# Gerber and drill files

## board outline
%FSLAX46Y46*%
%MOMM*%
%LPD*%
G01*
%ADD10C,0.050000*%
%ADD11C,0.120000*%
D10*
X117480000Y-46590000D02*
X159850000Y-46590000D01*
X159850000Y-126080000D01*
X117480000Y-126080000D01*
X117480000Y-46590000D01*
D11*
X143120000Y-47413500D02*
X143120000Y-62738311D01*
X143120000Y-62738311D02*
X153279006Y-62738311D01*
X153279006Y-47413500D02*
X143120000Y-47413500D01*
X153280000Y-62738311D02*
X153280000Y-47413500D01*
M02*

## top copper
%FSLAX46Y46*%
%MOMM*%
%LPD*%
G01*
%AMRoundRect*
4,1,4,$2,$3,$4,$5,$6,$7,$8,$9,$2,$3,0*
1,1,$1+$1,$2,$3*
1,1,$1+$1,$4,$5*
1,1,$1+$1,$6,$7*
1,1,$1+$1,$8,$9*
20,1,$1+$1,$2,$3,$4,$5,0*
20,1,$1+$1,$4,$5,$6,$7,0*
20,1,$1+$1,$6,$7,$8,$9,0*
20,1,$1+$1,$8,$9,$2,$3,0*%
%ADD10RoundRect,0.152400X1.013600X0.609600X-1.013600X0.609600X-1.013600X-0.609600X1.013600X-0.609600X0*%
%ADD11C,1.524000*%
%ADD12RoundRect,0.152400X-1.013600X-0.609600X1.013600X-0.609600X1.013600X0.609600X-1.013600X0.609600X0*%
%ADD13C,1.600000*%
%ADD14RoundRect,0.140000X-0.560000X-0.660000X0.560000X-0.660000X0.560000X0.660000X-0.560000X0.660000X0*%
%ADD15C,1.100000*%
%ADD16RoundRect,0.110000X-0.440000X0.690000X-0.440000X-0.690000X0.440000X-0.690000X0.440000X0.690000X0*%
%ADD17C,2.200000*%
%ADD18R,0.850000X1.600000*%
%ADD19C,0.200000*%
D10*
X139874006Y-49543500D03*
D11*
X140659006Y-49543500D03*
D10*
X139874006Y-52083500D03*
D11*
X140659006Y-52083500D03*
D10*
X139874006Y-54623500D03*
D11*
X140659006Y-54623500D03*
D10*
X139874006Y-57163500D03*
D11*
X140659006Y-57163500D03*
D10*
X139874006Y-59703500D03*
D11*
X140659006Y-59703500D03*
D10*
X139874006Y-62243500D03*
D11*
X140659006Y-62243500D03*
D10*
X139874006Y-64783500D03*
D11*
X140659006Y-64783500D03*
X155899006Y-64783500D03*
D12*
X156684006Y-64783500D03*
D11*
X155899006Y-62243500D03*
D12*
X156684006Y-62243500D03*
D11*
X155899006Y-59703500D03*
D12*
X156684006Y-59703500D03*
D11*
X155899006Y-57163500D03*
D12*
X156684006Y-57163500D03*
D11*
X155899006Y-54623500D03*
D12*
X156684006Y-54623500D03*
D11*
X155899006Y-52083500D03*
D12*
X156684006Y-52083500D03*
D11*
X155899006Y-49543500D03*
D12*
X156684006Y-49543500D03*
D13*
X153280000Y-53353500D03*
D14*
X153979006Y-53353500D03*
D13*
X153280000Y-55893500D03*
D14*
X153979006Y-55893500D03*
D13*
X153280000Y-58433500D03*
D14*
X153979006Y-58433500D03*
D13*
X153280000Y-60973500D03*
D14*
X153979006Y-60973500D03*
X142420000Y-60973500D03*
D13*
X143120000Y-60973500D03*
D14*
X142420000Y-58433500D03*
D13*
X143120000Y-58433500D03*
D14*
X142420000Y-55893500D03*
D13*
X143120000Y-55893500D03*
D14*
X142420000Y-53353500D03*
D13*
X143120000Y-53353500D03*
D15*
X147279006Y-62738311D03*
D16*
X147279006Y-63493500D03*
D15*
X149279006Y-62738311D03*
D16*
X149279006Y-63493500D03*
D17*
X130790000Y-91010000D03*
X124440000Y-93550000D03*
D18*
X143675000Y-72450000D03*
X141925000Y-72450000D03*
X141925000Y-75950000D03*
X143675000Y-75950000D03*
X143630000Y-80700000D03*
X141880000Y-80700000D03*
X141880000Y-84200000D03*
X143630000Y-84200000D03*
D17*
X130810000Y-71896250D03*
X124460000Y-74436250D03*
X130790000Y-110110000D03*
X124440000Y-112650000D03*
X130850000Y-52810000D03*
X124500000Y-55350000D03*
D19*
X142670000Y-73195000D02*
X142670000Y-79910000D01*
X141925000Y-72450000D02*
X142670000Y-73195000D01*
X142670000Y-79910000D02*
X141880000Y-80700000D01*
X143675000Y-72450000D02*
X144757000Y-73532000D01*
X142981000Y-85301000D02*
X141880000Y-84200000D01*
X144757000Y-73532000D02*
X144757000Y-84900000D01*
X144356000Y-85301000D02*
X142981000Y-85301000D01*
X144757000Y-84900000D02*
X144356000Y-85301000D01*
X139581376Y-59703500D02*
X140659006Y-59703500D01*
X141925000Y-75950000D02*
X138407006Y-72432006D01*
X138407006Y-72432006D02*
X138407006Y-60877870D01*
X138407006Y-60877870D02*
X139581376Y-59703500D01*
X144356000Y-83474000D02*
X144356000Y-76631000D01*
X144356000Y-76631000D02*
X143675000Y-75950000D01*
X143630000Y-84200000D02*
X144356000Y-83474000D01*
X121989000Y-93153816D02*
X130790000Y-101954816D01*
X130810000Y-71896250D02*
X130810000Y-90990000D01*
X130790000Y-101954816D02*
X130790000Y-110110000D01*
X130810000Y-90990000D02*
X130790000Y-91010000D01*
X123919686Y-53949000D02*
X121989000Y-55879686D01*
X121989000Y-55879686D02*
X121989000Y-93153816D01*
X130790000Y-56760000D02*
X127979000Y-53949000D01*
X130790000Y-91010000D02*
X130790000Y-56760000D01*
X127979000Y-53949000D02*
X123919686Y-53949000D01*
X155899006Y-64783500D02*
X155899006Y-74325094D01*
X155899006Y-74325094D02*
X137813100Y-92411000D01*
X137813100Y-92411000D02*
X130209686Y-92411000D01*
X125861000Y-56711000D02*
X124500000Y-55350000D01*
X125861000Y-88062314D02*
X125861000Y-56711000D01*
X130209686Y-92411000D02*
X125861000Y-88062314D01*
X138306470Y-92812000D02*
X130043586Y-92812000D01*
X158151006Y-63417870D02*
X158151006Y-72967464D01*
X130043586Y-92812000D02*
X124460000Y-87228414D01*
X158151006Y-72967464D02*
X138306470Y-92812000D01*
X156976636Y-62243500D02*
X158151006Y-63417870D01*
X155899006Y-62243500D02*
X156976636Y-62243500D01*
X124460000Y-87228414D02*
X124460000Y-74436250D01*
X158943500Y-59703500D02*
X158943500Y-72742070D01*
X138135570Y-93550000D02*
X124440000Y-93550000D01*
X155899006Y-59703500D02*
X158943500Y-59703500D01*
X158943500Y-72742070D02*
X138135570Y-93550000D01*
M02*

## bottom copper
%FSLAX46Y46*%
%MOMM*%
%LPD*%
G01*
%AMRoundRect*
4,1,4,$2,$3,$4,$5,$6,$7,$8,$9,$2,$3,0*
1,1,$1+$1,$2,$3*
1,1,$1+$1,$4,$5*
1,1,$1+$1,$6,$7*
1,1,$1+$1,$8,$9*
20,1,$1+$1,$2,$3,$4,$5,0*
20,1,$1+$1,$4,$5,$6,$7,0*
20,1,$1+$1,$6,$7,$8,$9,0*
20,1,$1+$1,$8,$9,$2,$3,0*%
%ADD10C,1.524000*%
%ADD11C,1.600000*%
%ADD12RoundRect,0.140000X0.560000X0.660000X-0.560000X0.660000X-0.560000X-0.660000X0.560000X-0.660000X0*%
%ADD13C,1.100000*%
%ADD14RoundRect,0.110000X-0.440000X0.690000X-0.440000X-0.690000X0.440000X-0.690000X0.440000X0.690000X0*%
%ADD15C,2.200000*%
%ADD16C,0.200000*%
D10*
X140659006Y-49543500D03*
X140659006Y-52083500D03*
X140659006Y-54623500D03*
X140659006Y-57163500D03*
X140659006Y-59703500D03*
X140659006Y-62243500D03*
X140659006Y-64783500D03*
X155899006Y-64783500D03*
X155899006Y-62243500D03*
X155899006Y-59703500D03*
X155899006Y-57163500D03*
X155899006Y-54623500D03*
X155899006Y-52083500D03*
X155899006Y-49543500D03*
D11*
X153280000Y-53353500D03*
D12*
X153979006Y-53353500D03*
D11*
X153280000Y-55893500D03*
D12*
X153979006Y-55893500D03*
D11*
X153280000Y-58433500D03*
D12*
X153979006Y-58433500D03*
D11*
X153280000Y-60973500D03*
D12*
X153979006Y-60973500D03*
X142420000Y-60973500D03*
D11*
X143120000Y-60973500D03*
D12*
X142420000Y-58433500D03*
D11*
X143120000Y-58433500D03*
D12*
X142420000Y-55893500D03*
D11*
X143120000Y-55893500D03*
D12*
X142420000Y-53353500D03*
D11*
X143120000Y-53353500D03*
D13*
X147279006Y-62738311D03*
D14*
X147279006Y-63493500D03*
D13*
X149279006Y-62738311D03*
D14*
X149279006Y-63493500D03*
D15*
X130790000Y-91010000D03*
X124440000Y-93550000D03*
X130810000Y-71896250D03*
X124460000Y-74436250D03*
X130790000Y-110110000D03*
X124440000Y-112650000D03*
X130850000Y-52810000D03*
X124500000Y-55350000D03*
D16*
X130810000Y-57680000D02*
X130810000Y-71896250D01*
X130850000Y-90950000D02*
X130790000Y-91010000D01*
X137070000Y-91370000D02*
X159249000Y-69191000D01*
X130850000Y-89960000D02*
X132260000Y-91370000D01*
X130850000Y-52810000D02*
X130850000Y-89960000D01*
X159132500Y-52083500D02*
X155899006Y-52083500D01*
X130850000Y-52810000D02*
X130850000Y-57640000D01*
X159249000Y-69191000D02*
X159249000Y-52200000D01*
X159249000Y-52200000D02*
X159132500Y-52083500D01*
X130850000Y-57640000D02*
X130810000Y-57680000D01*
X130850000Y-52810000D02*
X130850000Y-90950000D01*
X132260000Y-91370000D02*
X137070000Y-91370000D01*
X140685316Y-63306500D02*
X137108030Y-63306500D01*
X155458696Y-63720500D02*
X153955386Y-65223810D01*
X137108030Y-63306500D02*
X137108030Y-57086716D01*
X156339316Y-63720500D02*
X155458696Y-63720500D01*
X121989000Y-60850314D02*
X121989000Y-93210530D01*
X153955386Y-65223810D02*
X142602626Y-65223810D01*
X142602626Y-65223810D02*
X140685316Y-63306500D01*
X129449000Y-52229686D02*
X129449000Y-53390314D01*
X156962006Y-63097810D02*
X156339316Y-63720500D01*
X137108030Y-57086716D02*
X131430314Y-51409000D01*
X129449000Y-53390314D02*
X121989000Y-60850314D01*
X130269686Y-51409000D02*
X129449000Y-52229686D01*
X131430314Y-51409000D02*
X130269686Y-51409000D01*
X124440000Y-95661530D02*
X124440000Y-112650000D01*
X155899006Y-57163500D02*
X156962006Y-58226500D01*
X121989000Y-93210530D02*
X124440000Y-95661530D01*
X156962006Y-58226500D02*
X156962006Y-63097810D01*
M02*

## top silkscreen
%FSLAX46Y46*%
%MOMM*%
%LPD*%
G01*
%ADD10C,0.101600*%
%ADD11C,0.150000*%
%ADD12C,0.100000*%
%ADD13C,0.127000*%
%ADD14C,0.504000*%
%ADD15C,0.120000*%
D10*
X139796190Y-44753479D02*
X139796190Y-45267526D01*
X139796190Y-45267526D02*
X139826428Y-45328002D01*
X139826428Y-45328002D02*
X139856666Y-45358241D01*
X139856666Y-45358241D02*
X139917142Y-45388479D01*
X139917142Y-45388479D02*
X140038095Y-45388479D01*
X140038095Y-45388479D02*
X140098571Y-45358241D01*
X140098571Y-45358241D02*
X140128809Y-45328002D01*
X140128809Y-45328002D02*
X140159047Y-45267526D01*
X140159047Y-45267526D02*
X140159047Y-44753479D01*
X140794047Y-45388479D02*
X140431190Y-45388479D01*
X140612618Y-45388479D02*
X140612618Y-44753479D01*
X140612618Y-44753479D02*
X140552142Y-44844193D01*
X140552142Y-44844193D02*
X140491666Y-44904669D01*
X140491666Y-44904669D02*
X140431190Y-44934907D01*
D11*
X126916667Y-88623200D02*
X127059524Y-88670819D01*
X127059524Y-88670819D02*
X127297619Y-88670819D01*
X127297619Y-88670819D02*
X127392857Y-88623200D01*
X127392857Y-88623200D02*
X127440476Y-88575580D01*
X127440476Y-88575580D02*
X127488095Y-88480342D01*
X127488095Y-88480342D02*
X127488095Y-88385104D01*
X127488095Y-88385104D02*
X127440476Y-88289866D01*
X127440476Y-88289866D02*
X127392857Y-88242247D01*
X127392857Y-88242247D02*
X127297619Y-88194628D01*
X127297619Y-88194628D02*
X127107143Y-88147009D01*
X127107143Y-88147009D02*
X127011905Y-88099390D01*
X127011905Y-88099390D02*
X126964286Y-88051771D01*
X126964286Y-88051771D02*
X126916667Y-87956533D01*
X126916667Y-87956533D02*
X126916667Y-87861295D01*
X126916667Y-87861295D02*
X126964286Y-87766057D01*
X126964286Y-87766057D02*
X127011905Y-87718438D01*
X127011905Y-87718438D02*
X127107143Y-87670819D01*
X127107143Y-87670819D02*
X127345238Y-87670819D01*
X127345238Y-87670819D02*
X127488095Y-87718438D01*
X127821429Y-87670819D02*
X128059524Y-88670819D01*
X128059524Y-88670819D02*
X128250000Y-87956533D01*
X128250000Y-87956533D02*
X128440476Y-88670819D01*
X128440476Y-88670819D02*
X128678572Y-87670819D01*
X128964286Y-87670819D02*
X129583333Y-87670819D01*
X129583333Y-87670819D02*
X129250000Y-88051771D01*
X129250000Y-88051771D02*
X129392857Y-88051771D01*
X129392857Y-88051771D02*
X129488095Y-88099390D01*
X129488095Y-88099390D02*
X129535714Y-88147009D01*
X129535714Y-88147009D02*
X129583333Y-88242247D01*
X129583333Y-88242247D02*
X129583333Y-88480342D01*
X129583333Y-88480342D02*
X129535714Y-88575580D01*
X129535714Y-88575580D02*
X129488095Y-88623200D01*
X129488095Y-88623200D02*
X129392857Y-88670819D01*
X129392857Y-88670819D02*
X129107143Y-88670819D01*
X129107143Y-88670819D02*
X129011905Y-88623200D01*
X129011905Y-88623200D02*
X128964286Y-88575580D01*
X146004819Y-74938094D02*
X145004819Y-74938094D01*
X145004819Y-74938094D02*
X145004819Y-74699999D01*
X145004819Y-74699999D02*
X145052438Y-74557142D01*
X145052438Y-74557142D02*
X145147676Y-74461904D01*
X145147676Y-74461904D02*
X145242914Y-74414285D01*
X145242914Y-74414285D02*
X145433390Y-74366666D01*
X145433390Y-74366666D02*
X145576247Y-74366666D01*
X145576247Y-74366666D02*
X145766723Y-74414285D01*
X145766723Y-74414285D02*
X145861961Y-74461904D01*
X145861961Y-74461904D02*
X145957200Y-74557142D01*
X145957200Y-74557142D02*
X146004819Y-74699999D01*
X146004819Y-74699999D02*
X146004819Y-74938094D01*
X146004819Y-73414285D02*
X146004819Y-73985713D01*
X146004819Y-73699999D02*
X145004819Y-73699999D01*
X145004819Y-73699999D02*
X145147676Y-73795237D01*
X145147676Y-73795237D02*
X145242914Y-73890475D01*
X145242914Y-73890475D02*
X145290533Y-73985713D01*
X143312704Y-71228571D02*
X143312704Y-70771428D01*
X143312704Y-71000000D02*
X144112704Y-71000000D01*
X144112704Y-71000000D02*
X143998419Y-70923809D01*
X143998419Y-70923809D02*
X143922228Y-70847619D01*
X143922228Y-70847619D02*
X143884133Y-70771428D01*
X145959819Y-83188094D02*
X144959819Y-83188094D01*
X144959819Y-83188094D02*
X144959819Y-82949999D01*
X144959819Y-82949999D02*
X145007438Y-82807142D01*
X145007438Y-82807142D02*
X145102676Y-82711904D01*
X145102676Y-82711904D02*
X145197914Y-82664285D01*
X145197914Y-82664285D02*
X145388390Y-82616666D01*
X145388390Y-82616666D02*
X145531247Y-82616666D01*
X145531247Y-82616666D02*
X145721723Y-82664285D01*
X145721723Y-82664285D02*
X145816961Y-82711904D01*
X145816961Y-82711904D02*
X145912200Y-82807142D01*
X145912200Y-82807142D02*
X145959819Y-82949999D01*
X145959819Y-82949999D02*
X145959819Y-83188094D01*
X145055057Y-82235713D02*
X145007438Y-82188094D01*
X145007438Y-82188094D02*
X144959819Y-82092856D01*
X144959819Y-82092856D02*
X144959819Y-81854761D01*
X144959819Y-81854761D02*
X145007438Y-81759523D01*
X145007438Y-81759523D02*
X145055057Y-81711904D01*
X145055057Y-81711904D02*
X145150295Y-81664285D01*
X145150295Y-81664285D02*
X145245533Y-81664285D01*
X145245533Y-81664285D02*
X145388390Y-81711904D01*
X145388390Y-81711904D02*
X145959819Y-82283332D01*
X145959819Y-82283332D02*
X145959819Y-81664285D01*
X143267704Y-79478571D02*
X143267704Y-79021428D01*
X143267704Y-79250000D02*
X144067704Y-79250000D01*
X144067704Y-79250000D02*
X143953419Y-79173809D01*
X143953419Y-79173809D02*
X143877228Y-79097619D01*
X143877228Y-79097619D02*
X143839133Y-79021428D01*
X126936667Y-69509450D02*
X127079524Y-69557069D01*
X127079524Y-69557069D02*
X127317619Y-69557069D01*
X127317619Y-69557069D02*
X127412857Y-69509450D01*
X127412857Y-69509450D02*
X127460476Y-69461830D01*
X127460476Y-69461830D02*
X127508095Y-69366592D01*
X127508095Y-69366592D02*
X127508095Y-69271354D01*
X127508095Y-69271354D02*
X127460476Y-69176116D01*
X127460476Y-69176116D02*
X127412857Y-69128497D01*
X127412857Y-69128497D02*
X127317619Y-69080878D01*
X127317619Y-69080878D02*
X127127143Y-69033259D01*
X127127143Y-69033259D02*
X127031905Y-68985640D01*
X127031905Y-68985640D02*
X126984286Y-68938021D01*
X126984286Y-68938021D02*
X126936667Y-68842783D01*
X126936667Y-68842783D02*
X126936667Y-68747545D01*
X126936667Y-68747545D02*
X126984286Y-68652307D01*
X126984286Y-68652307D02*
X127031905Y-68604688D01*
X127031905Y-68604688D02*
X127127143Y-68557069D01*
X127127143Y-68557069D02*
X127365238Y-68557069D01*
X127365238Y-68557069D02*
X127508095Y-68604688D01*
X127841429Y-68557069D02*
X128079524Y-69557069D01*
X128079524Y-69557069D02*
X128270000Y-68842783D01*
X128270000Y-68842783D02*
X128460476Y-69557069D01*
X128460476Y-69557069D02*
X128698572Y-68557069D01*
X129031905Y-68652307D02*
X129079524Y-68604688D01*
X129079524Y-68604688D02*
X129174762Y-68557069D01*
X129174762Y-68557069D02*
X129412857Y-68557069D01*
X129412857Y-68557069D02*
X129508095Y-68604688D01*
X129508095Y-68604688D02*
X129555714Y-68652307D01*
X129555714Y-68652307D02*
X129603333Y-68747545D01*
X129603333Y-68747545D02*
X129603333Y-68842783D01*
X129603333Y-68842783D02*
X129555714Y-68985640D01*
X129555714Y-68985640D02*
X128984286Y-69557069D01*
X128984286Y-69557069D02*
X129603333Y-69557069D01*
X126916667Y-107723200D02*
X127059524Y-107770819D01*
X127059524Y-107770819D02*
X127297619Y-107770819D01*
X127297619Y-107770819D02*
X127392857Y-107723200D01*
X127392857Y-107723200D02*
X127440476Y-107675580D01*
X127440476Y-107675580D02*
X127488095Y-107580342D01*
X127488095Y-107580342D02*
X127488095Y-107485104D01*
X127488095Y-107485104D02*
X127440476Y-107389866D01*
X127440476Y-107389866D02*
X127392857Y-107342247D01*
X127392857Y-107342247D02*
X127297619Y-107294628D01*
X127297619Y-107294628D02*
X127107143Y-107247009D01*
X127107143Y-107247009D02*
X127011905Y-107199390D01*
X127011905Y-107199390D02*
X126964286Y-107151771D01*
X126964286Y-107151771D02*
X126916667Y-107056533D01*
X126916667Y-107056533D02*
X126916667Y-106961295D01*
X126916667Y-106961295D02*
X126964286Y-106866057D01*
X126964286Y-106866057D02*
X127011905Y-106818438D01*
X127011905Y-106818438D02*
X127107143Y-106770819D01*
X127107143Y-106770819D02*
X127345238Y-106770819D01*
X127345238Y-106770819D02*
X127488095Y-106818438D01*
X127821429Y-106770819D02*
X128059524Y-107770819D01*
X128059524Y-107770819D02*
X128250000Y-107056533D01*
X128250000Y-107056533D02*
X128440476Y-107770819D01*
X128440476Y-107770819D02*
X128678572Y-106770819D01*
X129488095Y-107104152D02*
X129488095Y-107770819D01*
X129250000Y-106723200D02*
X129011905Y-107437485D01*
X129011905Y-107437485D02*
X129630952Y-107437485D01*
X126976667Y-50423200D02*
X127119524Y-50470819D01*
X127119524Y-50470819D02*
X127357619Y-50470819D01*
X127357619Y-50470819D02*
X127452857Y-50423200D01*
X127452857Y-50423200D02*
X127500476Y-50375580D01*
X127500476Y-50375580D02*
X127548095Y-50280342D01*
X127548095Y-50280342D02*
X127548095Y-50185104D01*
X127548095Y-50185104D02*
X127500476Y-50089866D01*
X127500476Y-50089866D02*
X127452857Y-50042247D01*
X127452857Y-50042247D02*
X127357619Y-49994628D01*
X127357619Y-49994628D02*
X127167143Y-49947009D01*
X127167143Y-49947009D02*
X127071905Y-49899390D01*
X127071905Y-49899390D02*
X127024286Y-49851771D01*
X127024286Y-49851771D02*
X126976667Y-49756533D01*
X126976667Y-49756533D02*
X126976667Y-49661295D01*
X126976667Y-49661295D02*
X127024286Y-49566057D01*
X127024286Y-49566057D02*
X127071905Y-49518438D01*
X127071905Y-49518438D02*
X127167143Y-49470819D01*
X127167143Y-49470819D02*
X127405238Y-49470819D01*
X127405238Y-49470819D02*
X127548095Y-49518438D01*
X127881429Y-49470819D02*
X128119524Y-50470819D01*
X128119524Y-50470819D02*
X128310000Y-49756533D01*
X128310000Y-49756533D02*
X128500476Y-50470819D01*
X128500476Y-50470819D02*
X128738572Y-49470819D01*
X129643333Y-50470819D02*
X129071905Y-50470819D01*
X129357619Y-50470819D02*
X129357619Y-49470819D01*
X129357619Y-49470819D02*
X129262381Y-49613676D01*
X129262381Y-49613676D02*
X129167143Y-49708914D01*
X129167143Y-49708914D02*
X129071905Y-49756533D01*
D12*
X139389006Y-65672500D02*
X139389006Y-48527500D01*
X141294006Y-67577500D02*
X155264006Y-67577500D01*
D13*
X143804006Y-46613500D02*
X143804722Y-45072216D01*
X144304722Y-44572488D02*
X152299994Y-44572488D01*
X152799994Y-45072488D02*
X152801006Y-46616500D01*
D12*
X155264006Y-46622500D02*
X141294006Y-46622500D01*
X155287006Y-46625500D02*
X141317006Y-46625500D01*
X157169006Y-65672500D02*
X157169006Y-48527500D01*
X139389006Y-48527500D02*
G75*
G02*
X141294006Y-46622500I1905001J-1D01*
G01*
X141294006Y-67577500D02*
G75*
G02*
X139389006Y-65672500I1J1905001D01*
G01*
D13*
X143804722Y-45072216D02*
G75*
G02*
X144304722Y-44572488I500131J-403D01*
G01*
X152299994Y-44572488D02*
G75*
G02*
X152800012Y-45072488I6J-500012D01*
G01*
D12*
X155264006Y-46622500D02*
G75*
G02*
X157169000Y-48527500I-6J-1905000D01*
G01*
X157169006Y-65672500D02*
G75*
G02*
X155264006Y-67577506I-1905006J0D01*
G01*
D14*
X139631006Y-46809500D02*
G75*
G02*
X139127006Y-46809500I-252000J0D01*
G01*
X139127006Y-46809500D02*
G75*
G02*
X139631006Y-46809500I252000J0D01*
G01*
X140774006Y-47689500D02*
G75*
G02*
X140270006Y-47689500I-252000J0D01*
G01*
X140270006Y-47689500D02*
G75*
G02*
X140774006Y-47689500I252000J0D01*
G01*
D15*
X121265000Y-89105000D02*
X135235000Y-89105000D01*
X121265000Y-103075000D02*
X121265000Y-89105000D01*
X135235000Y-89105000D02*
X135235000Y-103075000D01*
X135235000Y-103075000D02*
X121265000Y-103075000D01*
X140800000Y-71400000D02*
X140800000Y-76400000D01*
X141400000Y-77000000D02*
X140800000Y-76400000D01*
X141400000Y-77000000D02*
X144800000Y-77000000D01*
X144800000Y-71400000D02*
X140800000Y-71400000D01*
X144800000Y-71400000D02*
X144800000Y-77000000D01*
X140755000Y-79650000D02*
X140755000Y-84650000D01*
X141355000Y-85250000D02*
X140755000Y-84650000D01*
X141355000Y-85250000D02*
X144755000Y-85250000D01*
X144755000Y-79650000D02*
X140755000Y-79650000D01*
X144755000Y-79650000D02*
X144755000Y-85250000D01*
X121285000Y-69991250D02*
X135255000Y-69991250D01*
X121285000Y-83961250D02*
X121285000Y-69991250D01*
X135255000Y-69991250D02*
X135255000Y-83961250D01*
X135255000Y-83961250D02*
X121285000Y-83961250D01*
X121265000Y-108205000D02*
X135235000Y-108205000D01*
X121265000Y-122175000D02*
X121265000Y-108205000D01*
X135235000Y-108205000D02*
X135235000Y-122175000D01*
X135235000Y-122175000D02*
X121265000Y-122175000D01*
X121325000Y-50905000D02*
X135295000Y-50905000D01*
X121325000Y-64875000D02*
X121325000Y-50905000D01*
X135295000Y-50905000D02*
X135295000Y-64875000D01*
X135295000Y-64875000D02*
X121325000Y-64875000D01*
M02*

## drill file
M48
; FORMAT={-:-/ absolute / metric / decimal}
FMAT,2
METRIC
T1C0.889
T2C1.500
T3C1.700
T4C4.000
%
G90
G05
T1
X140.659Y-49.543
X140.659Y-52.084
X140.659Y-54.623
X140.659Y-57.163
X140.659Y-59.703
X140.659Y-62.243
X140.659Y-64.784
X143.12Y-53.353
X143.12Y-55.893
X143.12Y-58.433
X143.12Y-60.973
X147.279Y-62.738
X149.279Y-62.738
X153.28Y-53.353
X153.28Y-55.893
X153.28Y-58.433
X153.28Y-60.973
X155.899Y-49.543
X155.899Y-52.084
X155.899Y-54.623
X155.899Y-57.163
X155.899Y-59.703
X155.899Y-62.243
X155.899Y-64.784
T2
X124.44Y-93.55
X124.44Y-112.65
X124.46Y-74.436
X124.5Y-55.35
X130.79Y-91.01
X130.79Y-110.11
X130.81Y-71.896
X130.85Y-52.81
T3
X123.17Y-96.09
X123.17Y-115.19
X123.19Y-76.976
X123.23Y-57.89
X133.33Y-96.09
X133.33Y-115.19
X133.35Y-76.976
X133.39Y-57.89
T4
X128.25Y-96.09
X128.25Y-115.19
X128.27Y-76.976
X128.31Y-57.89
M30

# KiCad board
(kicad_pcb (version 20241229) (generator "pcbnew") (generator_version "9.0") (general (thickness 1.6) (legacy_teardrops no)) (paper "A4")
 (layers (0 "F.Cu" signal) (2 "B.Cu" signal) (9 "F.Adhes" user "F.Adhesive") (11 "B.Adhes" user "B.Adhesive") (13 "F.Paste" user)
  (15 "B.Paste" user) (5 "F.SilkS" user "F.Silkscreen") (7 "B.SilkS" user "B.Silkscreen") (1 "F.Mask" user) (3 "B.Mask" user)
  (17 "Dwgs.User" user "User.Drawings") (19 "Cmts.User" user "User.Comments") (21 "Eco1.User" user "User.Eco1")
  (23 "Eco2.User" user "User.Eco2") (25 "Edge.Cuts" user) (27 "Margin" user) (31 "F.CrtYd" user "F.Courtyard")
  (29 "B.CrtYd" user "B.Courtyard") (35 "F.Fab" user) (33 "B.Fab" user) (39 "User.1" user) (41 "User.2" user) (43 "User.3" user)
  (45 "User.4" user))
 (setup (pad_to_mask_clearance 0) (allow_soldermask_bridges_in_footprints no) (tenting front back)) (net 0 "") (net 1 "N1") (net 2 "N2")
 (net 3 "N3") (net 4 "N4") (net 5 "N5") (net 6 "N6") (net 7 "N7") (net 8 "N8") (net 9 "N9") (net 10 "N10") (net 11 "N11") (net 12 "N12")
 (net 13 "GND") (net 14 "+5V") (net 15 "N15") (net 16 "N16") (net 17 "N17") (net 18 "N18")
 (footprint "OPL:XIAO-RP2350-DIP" (layer "F.Cu") (at 148.28 57.1)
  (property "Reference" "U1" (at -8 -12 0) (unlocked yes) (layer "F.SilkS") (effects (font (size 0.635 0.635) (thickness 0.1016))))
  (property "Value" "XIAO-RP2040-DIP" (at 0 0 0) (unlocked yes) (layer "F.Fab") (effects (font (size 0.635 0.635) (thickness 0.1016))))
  (fp_line (start -8.890994 8.5725) (end -8.890994 -8.5725) (stroke (width 0.1) (type solid)) (layer "F.SilkS"))
  (fp_line (start -6.985994 10.4775) (end 6.984006 10.4775) (stroke (width 0.1) (type solid)) (layer "F.SilkS"))
  (fp_line (start -4.475994 -10.4865) (end -4.475278 -12.027784) (stroke (width 0.127) (type solid)) (layer "F.SilkS"))
  (fp_line (start -3.975278 -12.527512) (end 4.019994 -12.527512) (stroke (width 0.127) (type solid)) (layer "F.SilkS"))
  (fp_line (start 4.519994 -12.027512) (end 4.521006 -10.4835) (stroke (width 0.127) (type solid)) (layer "F.SilkS"))
  (fp_line (start 6.984006 -10.4775) (end -6.985994 -10.4775) (stroke (width 0.1) (type solid)) (layer "F.SilkS"))
  (fp_line (start 7.007006 -10.4745) (end -6.962994 -10.4745) (stroke (width 0.1) (type solid)) (layer "F.SilkS"))
  (fp_line (start 8.889006 8.5725) (end 8.889006 -8.5725) (stroke (width 0.1) (type solid)) (layer "F.SilkS"))
  (fp_arc (start -8.890994 -8.5725) (mid -8.333032 -9.919538) (end -6.985994 -10.4775) (stroke (width 0.1) (type solid)) (layer "F.SilkS"))
  (fp_arc (start -6.985994 10.4775) (mid -8.333032 9.919538) (end -8.890994 8.5725) (stroke (width 0.1) (type solid)) (layer "F.SilkS"))
  (fp_arc (start -4.475278 -12.027784) (mid -4.328701 -12.381119) (end -3.975278 -12.527512) (stroke (width 0.127) (type default))
   (layer "F.SilkS"))
  (fp_arc (start 4.019994 -12.527512) (mid 4.373559 -12.38107) (end 4.519994 -12.027512) (stroke (width 0.127) (type default))
   (layer "F.SilkS"))
  (fp_arc (start 6.984006 -10.4775) (mid 8.331044 -9.919538) (end 8.889006 -8.5725) (stroke (width 0.1) (type solid)) (layer "F.SilkS"))
  (fp_arc (start 8.889006 8.5725) (mid 8.331044 9.919538) (end 6.984006 10.4775) (stroke (width 0.1) (type solid)) (layer "F.SilkS"))
  (fp_circle (center -8.900994 -10.2905) (end -8.900994 -10.5445) (stroke (width 0.5) (type solid)) (fill yes) (layer "F.SilkS"))
  (fp_circle (center -7.757994 -9.4105) (end -7.757994 -9.6645) (stroke (width 0.5) (type solid)) (fill yes) (layer "F.SilkS"))
  (fp_line (start -5.16 -9.6865) (end -5.16 5.638311) (stroke (width 0.12) (type default)) (layer "Edge.Cuts"))
  (fp_line (start -5.16 5.638311) (end 4.999006 5.638311) (stroke (width 0.12) (type default)) (layer "Edge.Cuts"))
  (fp_line (start 4.999006 -9.6865) (end -5.16 -9.6865) (stroke (width 0.12) (type default)) (layer "Edge.Cuts"))
  (fp_line (start 5 5.638311) (end 5 -9.6865) (stroke (width 0.12) (type default)) (layer "Edge.Cuts"))
  (pad "1" smd roundrect (at -8.405994 -7.5565 180) (size 2.332 1.524) (layers "F.Cu" "F.Mask") (roundrect_rratio 0.1) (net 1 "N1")
   (thermal_bridge_angle 45))
  (pad "1" thru_hole circle (at -7.620994 -7.5565 180) (size 1.524 1.524) (drill 0.889) (layers "*.Cu" "*.Mask") (remove_unused_layers no)
   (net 1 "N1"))
  (pad "2" smd roundrect (at -8.405994 -5.0165 180) (size 2.332 1.524) (layers "F.Cu" "F.Mask") (roundrect_rratio 0.1) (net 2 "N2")
   (thermal_bridge_angle 45))
  (pad "2" thru_hole circle (at -7.620994 -5.0165 180) (size 1.524 1.524) (drill 0.889) (layers "*.Cu" "*.Mask") (remove_unused_layers no)
   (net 2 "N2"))
  (pad "3" smd roundrect (at -8.405994 -2.4765 180) (size 2.332 1.524) (layers "F.Cu" "F.Mask") (roundrect_rratio 0.1) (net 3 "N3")
   (thermal_bridge_angle 45))
  (pad "3" thru_hole circle (at -7.620994 -2.4765 180) (size 1.524 1.524) (drill 0.889) (layers "*.Cu" "*.Mask") (remove_unused_layers no)
   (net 3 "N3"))
  (pad "4" smd roundrect (at -8.405994 0.0635 180) (size 2.332 1.524) (layers "F.Cu" "F.Mask") (roundrect_rratio 0.1) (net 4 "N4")
   (thermal_bridge_angle 45))
  (pad "4" thru_hole circle (at -7.620994 0.0635 180) (size 1.524 1.524) (drill 0.889) (layers "*.Cu" "*.Mask") (remove_unused_layers no)
   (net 4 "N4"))
  (pad "5" smd roundrect (at -8.405994 2.6035 180) (size 2.332 1.524) (layers "F.Cu" "F.Mask") (roundrect_rratio 0.1) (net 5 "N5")
   (thermal_bridge_angle 45))
  (pad "5" thru_hole circle (at -7.620994 2.6035 180) (size 1.524 1.524) (drill 0.889) (layers "*.Cu" "*.Mask") (remove_unused_layers no)
   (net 5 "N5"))
  (pad "6" smd roundrect (at -8.405994 5.1435 180) (size 2.332 1.524) (layers "F.Cu" "F.Mask") (roundrect_rratio 0.1) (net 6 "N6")
   (thermal_bridge_angle 45))
  (pad "6" thru_hole circle (at -7.620994 5.1435 180) (size 1.524 1.524) (drill 0.889) (layers "*.Cu" "*.Mask") (remove_unused_layers no)
   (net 6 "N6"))
  (pad "7" smd roundrect (at -8.405994 7.6835 180) (size 2.332 1.524) (layers "F.Cu" "F.Mask") (roundrect_rratio 0.1) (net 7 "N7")
   (thermal_bridge_angle 45))
  (pad "7" thru_hole circle (at -7.620994 7.6835 180) (size 1.524 1.524) (drill 0.889) (layers "*.Cu" "*.Mask") (remove_unused_layers no)
   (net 7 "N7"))
  (pad "8" thru_hole circle (at 7.619006 7.6835) (size 1.524 1.524) (drill 0.889) (layers "*.Cu" "*.Mask") (remove_unused_layers no)
   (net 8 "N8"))
  (pad "8" smd roundrect (at 8.404006 7.6835) (size 2.332 1.524) (layers "F.Cu" "F.Mask") (roundrect_rratio 0.1) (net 8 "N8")
   (thermal_bridge_angle 45))
  (pad "9" thru_hole circle (at 7.619006 5.1435) (size 1.524 1.524) (drill 0.889) (layers "*.Cu" "*.Mask") (remove_unused_layers no)
   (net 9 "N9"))
  (pad "9" smd roundrect (at 8.404006 5.1435) (size 2.332 1.524) (layers "F.Cu" "F.Mask") (roundrect_rratio 0.1) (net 9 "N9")
   (thermal_bridge_angle 45))
  (pad "10" thru_hole circle (at 7.619006 2.6035) (size 1.524 1.524) (drill 0.889) (layers "*.Cu" "*.Mask") (remove_unused_layers no)
   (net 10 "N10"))
  (pad "10" smd roundrect (at 8.404006 2.6035) (size 2.332 1.524) (layers "F.Cu" "F.Mask") (roundrect_rratio 0.1) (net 10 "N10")
   (thermal_bridge_angle 45))
  (pad "11" thru_hole circle (at 7.619006 0.0635) (size 1.524 1.524) (drill 0.889) (layers "*.Cu" "*.Mask") (remove_unused_layers no)
   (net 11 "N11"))
  (pad "11" smd roundrect (at 8.404006 0.0635) (size 2.332 1.524) (layers "F.Cu" "F.Mask") (roundrect_rratio 0.1) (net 11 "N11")
   (thermal_bridge_angle 45))
  (pad "12" thru_hole circle (at 7.619006 -2.4765) (size 1.524 1.524) (drill 0.889) (layers "*.Cu" "*.Mask") (remove_unused_layers no)
   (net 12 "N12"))
  (pad "12" smd roundrect (at 8.404006 -2.4765) (size 2.332 1.524) (layers "F.Cu" "F.Mask") (roundrect_rratio 0.1) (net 12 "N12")
   (thermal_bridge_angle 45))
  (pad "13" thru_hole circle (at 7.619006 -5.0165) (size 1.524 1.524) (drill 0.889) (layers "*.Cu" "*.Mask") (remove_unused_layers no)
   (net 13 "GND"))
  (pad "13" smd roundrect (at 8.404006 -5.0165) (size 2.332 1.524) (layers "F.Cu" "F.Mask") (roundrect_rratio 0.1) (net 13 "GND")
   (thermal_bridge_angle 45))
  (pad "14" thru_hole circle (at 7.619006 -7.5565) (size 1.524 1.524) (drill 0.889) (layers "*.Cu" "*.Mask") (remove_unused_layers no)
   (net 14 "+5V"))
  (pad "14" smd roundrect (at 8.404006 -7.5565) (size 2.332 1.524) (layers "F.Cu" "F.Mask") (roundrect_rratio 0.1) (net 14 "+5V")
   (thermal_bridge_angle 45))
  (pad "15" thru_hole circle (at 5 -3.7465 180) (size 1.6 1.6) (drill 0.889) (layers "*.Cu" "*.Mask") (remove_unused_layers no))
  (pad "15" smd roundrect (at 5.699006 -3.7465) (size 1.4 1.6) (layers "F.Cu" "F.Mask") (roundrect_rratio 0.1) (thermal_bridge_angle 45))
  (pad "15" smd roundrect (at 5.699006 -3.7465 180) (size 1.4 1.6) (layers "B.Cu" "B.Mask" "B.Paste") (roundrect_rratio 0.1)
   (thermal_bridge_angle 45))
  (pad "16" thru_hole circle (at 5 -1.2065 180) (size 1.6 1.6) (drill 0.889) (layers "*.Cu" "*.Mask") (remove_unused_layers no))
  (pad "16" smd roundrect (at 5.699006 -1.2065) (size 1.4 1.6) (layers "F.Cu" "F.Mask") (roundrect_rratio 0.1) (thermal_bridge_angle 45))
  (pad "16" smd roundrect (at 5.699006 -1.2065 180) (size 1.4 1.6) (layers "B.Cu" "B.Mask" "B.Paste") (roundrect_rratio 0.1)
   (thermal_bridge_angle 45))
  (pad "17" thru_hole circle (at 5 1.3335 180) (size 1.6 1.6) (drill 0.889) (layers "*.Cu" "*.Mask") (remove_unused_layers no))
  (pad "17" smd roundrect (at 5.699006 1.3335) (size 1.4 1.6) (layers "F.Cu" "F.Mask") (roundrect_rratio 0.1) (thermal_bridge_angle 45))
  (pad "17" smd roundrect (at 5.699006 1.3335 180) (size 1.4 1.6) (layers "B.Cu" "B.Mask" "B.Paste") (roundrect_rratio 0.1)
   (thermal_bridge_angle 45))
  (pad "18" thru_hole circle (at 5 3.8735 180) (size 1.6 1.6) (drill 0.889) (layers "*.Cu" "*.Mask") (remove_unused_layers no))
  (pad "18" smd roundrect (at 5.699006 3.8735) (size 1.4 1.6) (layers "F.Cu" "F.Mask") (roundrect_rratio 0.1) (thermal_bridge_angle 45))
  (pad "18" smd roundrect (at 5.699006 3.8735 180) (size 1.4 1.6) (layers "B.Cu" "B.Mask" "B.Paste") (roundrect_rratio 0.1)
   (thermal_bridge_angle 45))
  (pad "19" smd roundrect (at -5.86 3.8735) (size 1.4 1.6) (layers "F.Cu" "F.Mask") (roundrect_rratio 0.1) (thermal_bridge_angle 45))
  (pad "19" smd roundrect (at -5.86 3.8735 180) (size 1.4 1.6) (layers "B.Cu" "B.Mask" "B.Paste") (roundrect_rratio 0.1)
   (thermal_bridge_angle 45))
  (pad "19" thru_hole circle (at -5.16 3.8735 180) (size 1.6 1.6) (drill 0.889) (layers "*.Cu" "*.Mask") (remove_unused_layers no))
  (pad "20" smd roundrect (at -5.86 1.3335) (size 1.4 1.6) (layers "F.Cu" "F.Mask") (roundrect_rratio 0.1) (thermal_bridge_angle 45))
  (pad "20" smd roundrect (at -5.86 1.3335 180) (size 1.4 1.6) (layers "B.Cu" "B.Mask" "B.Paste") (roundrect_rratio 0.1)
   (thermal_bridge_angle 45))
  (pad "20" thru_hole circle (at -5.16 1.3335 180) (size 1.6 1.6) (drill 0.889) (layers "*.Cu" "*.Mask") (remove_unused_layers no))
  (pad "21" smd roundrect (at -5.86 -1.2065) (size 1.4 1.6) (layers "F.Cu" "F.Mask") (roundrect_rratio 0.1) (thermal_bridge_angle 45))
  (pad "21" smd roundrect (at -5.86 -1.2065 180) (size 1.4 1.6) (layers "B.Cu" "B.Mask" "B.Paste") (roundrect_rratio 0.1)
   (thermal_bridge_angle 45))
  (pad "21" thru_hole circle (at -5.16 -1.2065 180) (size 1.6 1.6) (drill 0.889) (layers "*.Cu" "*.Mask") (remove_unused_layers no))
  (pad "22" smd roundrect (at -5.86 -3.7465) (size 1.4 1.6) (layers "F.Cu" "F.Mask") (roundrect_rratio 0.1) (thermal_bridge_angle 45))
  (pad "22" smd roundrect (at -5.86 -3.7465 180) (size 1.4 1.6) (layers "B.Cu" "B.Mask" "B.Paste") (roundrect_rratio 0.1)
   (thermal_bridge_angle 45))
  (pad "22" thru_hole circle (at -5.16 -3.7465 180) (size 1.6 1.6) (drill 0.889) (layers "*.Cu" "*.Mask") (remove_unused_layers no))
  (pad "23" thru_hole circle (at -1.000994 5.638311 180) (size 1.1 1.1) (drill 0.889) (layers "*.Cu" "*.Mask") (remove_unused_layers no))
  (pad "23" smd roundrect (at -1.000994 6.3935 270) (size 1.6 1.1) (layers "F.Cu" "F.Mask") (roundrect_rratio 0.1) (thermal_bridge_angle 45))
  (pad "23" smd roundrect (at -1.000994 6.3935 270) (size 1.6 1.1) (layers "B.Cu" "B.Mask" "B.Paste") (roundrect_rratio 0.1)
   (thermal_bridge_angle 45))
  (pad "24" thru_hole circle (at 0.999006 5.638311 180) (size 1.1 1.1) (drill 0.889) (layers "*.Cu" "*.Mask") (remove_unused_layers no))
  (pad "24" smd roundrect (at 0.999006 6.3935 270) (size 1.6 1.1) (layers "F.Cu" "F.Mask") (roundrect_rratio 0.1) (thermal_bridge_angle 45))
  (pad "24" smd roundrect (at 0.999006 6.3935 270) (size 1.6 1.1) (layers "B.Cu" "B.Mask" "B.Paste") (roundrect_rratio 0.1)
   (thermal_bridge_angle 45)))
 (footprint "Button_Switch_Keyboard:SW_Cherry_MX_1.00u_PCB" (layer "F.Cu") (at 130.79 91.01)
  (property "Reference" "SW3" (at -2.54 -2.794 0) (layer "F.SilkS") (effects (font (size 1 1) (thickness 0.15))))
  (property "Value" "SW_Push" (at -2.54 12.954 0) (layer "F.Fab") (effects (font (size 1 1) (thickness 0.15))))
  (fp_line (start -9.525 -1.905) (end 4.445 -1.905) (stroke (width 0.12) (type solid)) (layer "F.SilkS"))
  (fp_line (start -9.525 12.065) (end -9.525 -1.905) (stroke (width 0.12) (type solid)) (layer "F.SilkS"))
  (fp_line (start 4.445 -1.905) (end 4.445 12.065) (stroke (width 0.12) (type solid)) (layer "F.SilkS"))
  (fp_line (start 4.445 12.065) (end -9.525 12.065) (stroke (width 0.12) (type solid)) (layer "F.SilkS"))
  (pad "" np_thru_hole circle (at -7.62 5.08) (size 1.7 1.7) (drill 1.7) (layers "*.Cu" "*.Mask"))
  (pad "" np_thru_hole circle (at -2.54 5.08) (size 4 4) (drill 4) (layers "*.Cu" "*.Mask"))
  (pad "" np_thru_hole circle (at 2.54 5.08) (size 1.7 1.7) (drill 1.7) (layers "*.Cu" "*.Mask"))
  (pad "1" thru_hole circle (at 0 0) (size 2.2 2.2) (drill 1.5) (layers "*.Cu" "*.Mask") (remove_unused_layers no) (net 13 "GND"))
  (pad "2" thru_hole circle (at -6.35 2.54) (size 2.2 2.2) (drill 1.5) (layers "*.Cu" "*.Mask") (remove_unused_layers no) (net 10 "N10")))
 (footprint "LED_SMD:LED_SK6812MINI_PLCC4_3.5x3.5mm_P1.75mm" (layer "F.Cu") (at 142.8 74.2 -90)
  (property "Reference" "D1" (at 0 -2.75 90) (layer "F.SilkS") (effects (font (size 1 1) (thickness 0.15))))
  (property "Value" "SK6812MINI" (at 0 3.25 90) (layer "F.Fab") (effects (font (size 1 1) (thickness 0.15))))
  (fp_line (start -2.8 2) (end 2.2 2) (stroke (width 0.12) (type solid)) (layer "F.SilkS"))
  (fp_line (start 2.8 1.4) (end 2.2 2) (stroke (width 0.12) (type default)) (layer "F.SilkS"))
  (fp_line (start 2.8 1.4) (end 2.8 -2) (stroke (width 0.12) (type solid)) (layer "F.SilkS"))
  (fp_line (start -2.8 -2) (end -2.8 2) (stroke (width 0.12) (type default)) (layer "F.SilkS"))
  (fp_line (start -2.8 -2) (end 2.8 -2) (stroke (width 0.12) (type solid)) (layer "F.SilkS"))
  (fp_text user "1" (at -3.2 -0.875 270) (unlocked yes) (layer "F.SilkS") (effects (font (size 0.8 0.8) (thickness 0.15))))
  (pad "1" smd rect (at -1.75 -0.875 270) (size 1.6 0.85) (layers "F.Cu" "F.Mask" "F.Paste") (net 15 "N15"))
  (pad "2" smd rect (at -1.75 0.875 270) (size 1.6 0.85) (layers "F.Cu" "F.Mask" "F.Paste") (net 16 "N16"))
  (pad "3" smd rect (at 1.75 0.875 270) (size 1.6 0.85) (layers "F.Cu" "F.Mask" "F.Paste") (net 5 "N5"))
  (pad "4" smd rect (at 1.75 -0.875 270) (size 1.6 0.85) (layers "F.Cu" "F.Mask" "F.Paste") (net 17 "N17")))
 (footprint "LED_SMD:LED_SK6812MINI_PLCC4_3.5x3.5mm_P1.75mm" (layer "F.Cu") (at 142.755 82.45 -90)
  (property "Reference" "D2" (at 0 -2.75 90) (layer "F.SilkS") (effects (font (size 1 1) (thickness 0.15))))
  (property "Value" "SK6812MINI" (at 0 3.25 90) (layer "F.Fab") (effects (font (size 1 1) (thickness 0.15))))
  (fp_line (start -2.8 2) (end 2.2 2) (stroke (width 0.12) (type solid)) (layer "F.SilkS"))
  (fp_line (start 2.8 1.4) (end 2.2 2) (stroke (width 0.12) (type default)) (layer "F.SilkS"))
  (fp_line (start 2.8 1.4) (end 2.8 -2) (stroke (width 0.12) (type solid)) (layer "F.SilkS"))
  (fp_line (start -2.8 -2) (end -2.8 2) (stroke (width 0.12) (type default)) (layer "F.SilkS"))
  (fp_line (start -2.8 -2) (end 2.8 -2) (stroke (width 0.12) (type solid)) (layer "F.SilkS"))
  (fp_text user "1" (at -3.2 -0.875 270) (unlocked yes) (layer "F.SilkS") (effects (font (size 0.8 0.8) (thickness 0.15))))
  (pad "1" smd rect (at -1.75 -0.875 270) (size 1.6 0.85) (layers "F.Cu" "F.Mask" "F.Paste") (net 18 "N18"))
  (pad "2" smd rect (at -1.75 0.875 270) (size 1.6 0.85) (layers "F.Cu" "F.Mask" "F.Paste") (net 16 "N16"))
  (pad "3" smd rect (at 1.75 0.875 270) (size 1.6 0.85) (layers "F.Cu" "F.Mask" "F.Paste") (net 15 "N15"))
  (pad "4" smd rect (at 1.75 -0.875 270) (size 1.6 0.85) (layers "F.Cu" "F.Mask" "F.Paste") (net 17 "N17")))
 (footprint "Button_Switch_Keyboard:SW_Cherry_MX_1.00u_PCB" (layer "F.Cu") (at 130.81 71.89625)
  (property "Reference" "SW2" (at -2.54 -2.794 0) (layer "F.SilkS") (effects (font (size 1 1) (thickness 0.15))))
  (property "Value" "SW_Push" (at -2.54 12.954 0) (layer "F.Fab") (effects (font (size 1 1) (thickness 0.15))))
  (fp_line (start -9.525 -1.905) (end 4.445 -1.905) (stroke (width 0.12) (type solid)) (layer "F.SilkS"))
  (fp_line (start -9.525 12.065) (end -9.525 -1.905) (stroke (width 0.12) (type solid)) (layer "F.SilkS"))
  (fp_line (start 4.445 -1.905) (end 4.445 12.065) (stroke (width 0.12) (type solid)) (layer "F.SilkS"))
  (fp_line (start 4.445 12.065) (end -9.525 12.065) (stroke (width 0.12) (type solid)) (layer "F.SilkS"))
  (pad "" np_thru_hole circle (at -7.62 5.08) (size 1.7 1.7) (drill 1.7) (layers "*.Cu" "*.Mask"))
  (pad "" np_thru_hole circle (at -2.54 5.08) (size 4 4) (drill 4) (layers "*.Cu" "*.Mask"))
  (pad "" np_thru_hole circle (at 2.54 5.08) (size 1.7 1.7) (drill 1.7) (layers "*.Cu" "*.Mask"))
  (pad "1" thru_hole circle (at 0 0) (size 2.2 2.2) (drill 1.5) (layers "*.Cu" "*.Mask") (remove_unused_layers no) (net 13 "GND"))
  (pad "2" thru_hole circle (at -6.35 2.54) (size 2.2 2.2) (drill 1.5) (layers "*.Cu" "*.Mask") (remove_unused_layers no) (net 9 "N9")))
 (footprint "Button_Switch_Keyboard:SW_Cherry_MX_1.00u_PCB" (layer "F.Cu") (at 130.79 110.11)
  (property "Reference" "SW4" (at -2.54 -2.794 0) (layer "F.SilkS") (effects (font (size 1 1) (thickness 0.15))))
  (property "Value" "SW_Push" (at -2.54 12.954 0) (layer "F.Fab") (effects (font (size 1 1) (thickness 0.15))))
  (fp_line (start -9.525 -1.905) (end 4.445 -1.905) (stroke (width 0.12) (type solid)) (layer "F.SilkS"))
  (fp_line (start -9.525 12.065) (end -9.525 -1.905) (stroke (width 0.12) (type solid)) (layer "F.SilkS"))
  (fp_line (start 4.445 -1.905) (end 4.445 12.065) (stroke (width 0.12) (type solid)) (layer "F.SilkS"))
  (fp_line (start 4.445 12.065) (end -9.525 12.065) (stroke (width 0.12) (type solid)) (layer "F.SilkS"))
  (pad "" np_thru_hole circle (at -7.62 5.08) (size 1.7 1.7) (drill 1.7) (layers "*.Cu" "*.Mask"))
  (pad "" np_thru_hole circle (at -2.54 5.08) (size 4 4) (drill 4) (layers "*.Cu" "*.Mask"))
  (pad "" np_thru_hole circle (at 2.54 5.08) (size 1.7 1.7) (drill 1.7) (layers "*.Cu" "*.Mask"))
  (pad "1" thru_hole circle (at 0 0) (size 2.2 2.2) (drill 1.5) (layers "*.Cu" "*.Mask") (remove_unused_layers no) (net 13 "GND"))
  (pad "2" thru_hole circle (at -6.35 2.54) (size 2.2 2.2) (drill 1.5) (layers "*.Cu" "*.Mask") (remove_unused_layers no) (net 11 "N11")))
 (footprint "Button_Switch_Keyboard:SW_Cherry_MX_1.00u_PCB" (layer "F.Cu") (at 130.85 52.81)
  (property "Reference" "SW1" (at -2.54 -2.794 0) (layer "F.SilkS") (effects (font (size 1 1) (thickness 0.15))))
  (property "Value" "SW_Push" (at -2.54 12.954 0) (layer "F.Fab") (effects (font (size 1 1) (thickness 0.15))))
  (fp_line (start -9.525 -1.905) (end 4.445 -1.905) (stroke (width 0.12) (type solid)) (layer "F.SilkS"))
  (fp_line (start -9.525 12.065) (end -9.525 -1.905) (stroke (width 0.12) (type solid)) (layer "F.SilkS"))
  (fp_line (start 4.445 -1.905) (end 4.445 12.065) (stroke (width 0.12) (type solid)) (layer "F.SilkS"))
  (fp_line (start 4.445 12.065) (end -9.525 12.065) (stroke (width 0.12) (type solid)) (layer "F.SilkS"))
  (pad "" np_thru_hole circle (at -7.62 5.08) (size 1.7 1.7) (drill 1.7) (layers "*.Cu" "*.Mask"))
  (pad "" np_thru_hole circle (at -2.54 5.08) (size 4 4) (drill 4) (layers "*.Cu" "*.Mask"))
  (pad "" np_thru_hole circle (at 2.54 5.08) (size 1.7 1.7) (drill 1.7) (layers "*.Cu" "*.Mask"))
  (pad "1" thru_hole circle (at 0 0) (size 2.2 2.2) (drill 1.5) (layers "*.Cu" "*.Mask") (remove_unused_layers no) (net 13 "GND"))
  (pad "2" thru_hole circle (at -6.35 2.54) (size 2.2 2.2) (drill 1.5) (layers "*.Cu" "*.Mask") (remove_unused_layers no) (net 8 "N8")))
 (gr_rect (start 117.48 46.59) (end 159.85 126.08) (stroke (width 0.05) (type default)) (fill no) (layer "Edge.Cuts"))
 (segment (start 142.67 73.195) (end 142.67 79.91) (width 0.2) (layer "F.Cu") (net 16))
 (segment (start 141.925 72.45) (end 142.67 73.195) (width 0.2) (layer "F.Cu") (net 16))
 (segment (start 142.67 79.91) (end 141.88 80.7) (width 0.2) (layer "F.Cu") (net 16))
 (segment (start 143.675 72.45) (end 144.757 73.532) (width 0.2) (layer "F.Cu") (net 15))
 (segment (start 142.981 85.301) (end 141.88 84.2) (width 0.2) (layer "F.Cu") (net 15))
 (segment (start 144.757 73.532) (end 144.757 84.9) (width 0.2) (layer "F.Cu") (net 15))
 (segment (start 144.356 85.301) (end 142.981 85.301) (width 0.2) (layer "F.Cu") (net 15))
 (segment (start 144.757 84.9) (end 144.356 85.301) (width 0.2) (layer "F.Cu") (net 15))
 (segment (start 139.581376 59.7035) (end 140.659006 59.7035) (width 0.2) (layer "F.Cu") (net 5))
 (segment (start 141.925 75.95) (end 138.407006 72.432006) (width 0.2) (layer "F.Cu") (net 5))
 (segment (start 138.407006 72.432006) (end 138.407006 60.87787) (width 0.2) (layer "F.Cu") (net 5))
 (segment (start 138.407006 60.87787) (end 139.581376 59.7035) (width 0.2) (layer "F.Cu") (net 5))
 (segment (start 144.356 83.474) (end 144.356 76.631) (width 0.2) (layer "F.Cu") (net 17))
 (segment (start 144.356 76.631) (end 143.675 75.95) (width 0.2) (layer "F.Cu") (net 17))
 (segment (start 143.63 84.2) (end 144.356 83.474) (width 0.2) (layer "F.Cu") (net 17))
 (segment (start 121.989 93.153816) (end 130.79 101.954816) (width 0.2) (layer "F.Cu") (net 13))
 (segment (start 130.81 71.89625) (end 130.81 90.99) (width 0.2) (layer "F.Cu") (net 13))
 (segment (start 130.79 101.954816) (end 130.79 110.11) (width 0.2) (layer "F.Cu") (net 13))
 (segment (start 130.81 90.99) (end 130.79 91.01) (width 0.2) (layer "F.Cu") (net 13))
 (segment (start 123.919686 53.949) (end 121.989 55.879686) (width 0.2) (layer "F.Cu") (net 13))
 (segment (start 121.989 55.879686) (end 121.989 93.153816) (width 0.2) (layer "F.Cu") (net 13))
 (segment (start 130.79 56.76) (end 127.979 53.949) (width 0.2) (layer "F.Cu") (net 13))
 (segment (start 130.79 91.01) (end 130.79 56.76) (width 0.2) (layer "F.Cu") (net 13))
 (segment (start 127.979 53.949) (end 123.919686 53.949) (width 0.2) (layer "F.Cu") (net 13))
 (segment (start 130.81 57.68) (end 130.81 71.89625) (width 0.2) (layer "B.Cu") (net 13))
 (segment (start 130.85 90.95) (end 130.79 91.01) (width 0.2) (layer "B.Cu") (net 13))
 (segment (start 137.07 91.37) (end 159.249 69.191) (width 0.2) (layer "B.Cu") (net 13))
 (segment (start 130.85 89.96) (end 132.26 91.37) (width 0.2) (layer "B.Cu") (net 13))
 (segment (start 130.85 52.81) (end 130.85 89.96) (width 0.2) (layer "B.Cu") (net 13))
 (segment (start 159.1325 52.0835) (end 155.899006 52.0835) (width 0.2) (layer "B.Cu") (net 13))
 (segment (start 130.85 52.81) (end 130.85 57.64) (width 0.2) (layer "B.Cu") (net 13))
 (segment (start 159.249 69.191) (end 159.249 52.2) (width 0.2) (layer "B.Cu") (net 13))
 (segment (start 159.249 52.2) (end 159.1325 52.0835) (width 0.2) (layer "B.Cu") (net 13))
 (segment (start 130.85 57.64) (end 130.81 57.68) (width 0.2) (layer "B.Cu") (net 13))
 (segment (start 130.85 52.81) (end 130.85 90.95) (width 0.2) (layer "B.Cu") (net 13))
 (segment (start 132.26 91.37) (end 137.07 91.37) (width 0.2) (layer "B.Cu") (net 13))
 (segment (start 155.899006 64.7835) (end 155.899006 74.325094) (width 0.2) (layer "F.Cu") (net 8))
 (segment (start 155.899006 74.325094) (end 137.8131 92.411) (width 0.2) (layer "F.Cu") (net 8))
 (segment (start 137.8131 92.411) (end 130.209686 92.411) (width 0.2) (layer "F.Cu") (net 8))
 (segment (start 125.861 56.711) (end 124.5 55.35) (width 0.2) (layer "F.Cu") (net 8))
 (segment (start 125.861 88.062314) (end 125.861 56.711) (width 0.2) (layer "F.Cu") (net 8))
 (segment (start 130.209686 92.411) (end 125.861 88.062314) (width 0.2) (layer "F.Cu") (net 8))
 (segment (start 138.30647 92.812) (end 130.043586 92.812) (width 0.2) (layer "F.Cu") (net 9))
 (segment (start 158.151006 63.41787) (end 158.151006 72.967464) (width 0.2) (layer "F.Cu") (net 9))
 (segment (start 130.043586 92.812) (end 124.46 87.228414) (width 0.2) (layer "F.Cu") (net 9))
 (segment (start 158.151006 72.967464) (end 138.30647 92.812) (width 0.2) (layer "F.Cu") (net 9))
 (segment (start 156.976636 62.2435) (end 158.151006 63.41787) (width 0.2) (layer "F.Cu") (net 9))
 (segment (start 155.899006 62.2435) (end 156.976636 62.2435) (width 0.2) (layer "F.Cu") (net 9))
 (segment (start 124.46 87.228414) (end 124.46 74.43625) (width 0.2) (layer "F.Cu") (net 9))
 (segment (start 158.9435 59.7035) (end 158.9435 72.74207) (width 0.2) (layer "F.Cu") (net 10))
 (segment (start 138.13557 93.55) (end 124.44 93.55) (width 0.2) (layer "F.Cu") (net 10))
 (segment (start 155.899006 59.7035) (end 158.9435 59.7035) (width 0.2) (layer "F.Cu") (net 10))
 (segment (start 158.9435 72.74207) (end 138.13557 93.55) (width 0.2) (layer "F.Cu") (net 10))
 (segment (start 140.685316 63.3065) (end 137.10803 63.3065) (width 0.2) (layer "B.Cu") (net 11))
 (segment (start 155.458696 63.7205) (end 153.955386 65.22381) (width 0.2) (layer "B.Cu") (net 11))
 (segment (start 137.10803 63.3065) (end 137.10803 57.086716) (width 0.2) (layer "B.Cu") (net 11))
 (segment (start 156.339316 63.7205) (end 155.458696 63.7205) (width 0.2) (layer "B.Cu") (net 11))
 (segment (start 121.989 60.850314) (end 121.989 93.21053) (width 0.2) (layer "B.Cu") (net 11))
 (segment (start 153.955386 65.22381) (end 142.602626 65.22381) (width 0.2) (layer "B.Cu") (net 11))
 (segment (start 142.602626 65.22381) (end 140.685316 63.3065) (width 0.2) (layer "B.Cu") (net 11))
 (segment (start 129.449 52.229686) (end 129.449 53.390314) (width 0.2) (layer "B.Cu") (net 11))
 (segment (start 156.962006 63.09781) (end 156.339316 63.7205) (width 0.2) (layer "B.Cu") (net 11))
 (segment (start 137.10803 57.086716) (end 131.430314 51.409) (width 0.2) (layer "B.Cu") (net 11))
 (segment (start 129.449 53.390314) (end 121.989 60.850314) (width 0.2) (layer "B.Cu") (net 11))
 (segment (start 130.269686 51.409) (end 129.449 52.229686) (width 0.2) (layer "B.Cu") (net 11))
 (segment (start 131.430314 51.409) (end 130.269686 51.409) (width 0.2) (layer "B.Cu") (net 11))
 (segment (start 124.44 95.66153) (end 124.44 112.65) (width 0.2) (layer "B.Cu") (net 11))
 (segment (start 155.899006 57.1635) (end 156.962006 58.2265) (width 0.2) (layer "B.Cu") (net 11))
 (segment (start 121.989 93.21053) (end 124.44 95.66153) (width 0.2) (layer "B.Cu") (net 11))
 (segment (start 156.962006 58.2265) (end 156.962006 63.09781) (width 0.2) (layer "B.Cu") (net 11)))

